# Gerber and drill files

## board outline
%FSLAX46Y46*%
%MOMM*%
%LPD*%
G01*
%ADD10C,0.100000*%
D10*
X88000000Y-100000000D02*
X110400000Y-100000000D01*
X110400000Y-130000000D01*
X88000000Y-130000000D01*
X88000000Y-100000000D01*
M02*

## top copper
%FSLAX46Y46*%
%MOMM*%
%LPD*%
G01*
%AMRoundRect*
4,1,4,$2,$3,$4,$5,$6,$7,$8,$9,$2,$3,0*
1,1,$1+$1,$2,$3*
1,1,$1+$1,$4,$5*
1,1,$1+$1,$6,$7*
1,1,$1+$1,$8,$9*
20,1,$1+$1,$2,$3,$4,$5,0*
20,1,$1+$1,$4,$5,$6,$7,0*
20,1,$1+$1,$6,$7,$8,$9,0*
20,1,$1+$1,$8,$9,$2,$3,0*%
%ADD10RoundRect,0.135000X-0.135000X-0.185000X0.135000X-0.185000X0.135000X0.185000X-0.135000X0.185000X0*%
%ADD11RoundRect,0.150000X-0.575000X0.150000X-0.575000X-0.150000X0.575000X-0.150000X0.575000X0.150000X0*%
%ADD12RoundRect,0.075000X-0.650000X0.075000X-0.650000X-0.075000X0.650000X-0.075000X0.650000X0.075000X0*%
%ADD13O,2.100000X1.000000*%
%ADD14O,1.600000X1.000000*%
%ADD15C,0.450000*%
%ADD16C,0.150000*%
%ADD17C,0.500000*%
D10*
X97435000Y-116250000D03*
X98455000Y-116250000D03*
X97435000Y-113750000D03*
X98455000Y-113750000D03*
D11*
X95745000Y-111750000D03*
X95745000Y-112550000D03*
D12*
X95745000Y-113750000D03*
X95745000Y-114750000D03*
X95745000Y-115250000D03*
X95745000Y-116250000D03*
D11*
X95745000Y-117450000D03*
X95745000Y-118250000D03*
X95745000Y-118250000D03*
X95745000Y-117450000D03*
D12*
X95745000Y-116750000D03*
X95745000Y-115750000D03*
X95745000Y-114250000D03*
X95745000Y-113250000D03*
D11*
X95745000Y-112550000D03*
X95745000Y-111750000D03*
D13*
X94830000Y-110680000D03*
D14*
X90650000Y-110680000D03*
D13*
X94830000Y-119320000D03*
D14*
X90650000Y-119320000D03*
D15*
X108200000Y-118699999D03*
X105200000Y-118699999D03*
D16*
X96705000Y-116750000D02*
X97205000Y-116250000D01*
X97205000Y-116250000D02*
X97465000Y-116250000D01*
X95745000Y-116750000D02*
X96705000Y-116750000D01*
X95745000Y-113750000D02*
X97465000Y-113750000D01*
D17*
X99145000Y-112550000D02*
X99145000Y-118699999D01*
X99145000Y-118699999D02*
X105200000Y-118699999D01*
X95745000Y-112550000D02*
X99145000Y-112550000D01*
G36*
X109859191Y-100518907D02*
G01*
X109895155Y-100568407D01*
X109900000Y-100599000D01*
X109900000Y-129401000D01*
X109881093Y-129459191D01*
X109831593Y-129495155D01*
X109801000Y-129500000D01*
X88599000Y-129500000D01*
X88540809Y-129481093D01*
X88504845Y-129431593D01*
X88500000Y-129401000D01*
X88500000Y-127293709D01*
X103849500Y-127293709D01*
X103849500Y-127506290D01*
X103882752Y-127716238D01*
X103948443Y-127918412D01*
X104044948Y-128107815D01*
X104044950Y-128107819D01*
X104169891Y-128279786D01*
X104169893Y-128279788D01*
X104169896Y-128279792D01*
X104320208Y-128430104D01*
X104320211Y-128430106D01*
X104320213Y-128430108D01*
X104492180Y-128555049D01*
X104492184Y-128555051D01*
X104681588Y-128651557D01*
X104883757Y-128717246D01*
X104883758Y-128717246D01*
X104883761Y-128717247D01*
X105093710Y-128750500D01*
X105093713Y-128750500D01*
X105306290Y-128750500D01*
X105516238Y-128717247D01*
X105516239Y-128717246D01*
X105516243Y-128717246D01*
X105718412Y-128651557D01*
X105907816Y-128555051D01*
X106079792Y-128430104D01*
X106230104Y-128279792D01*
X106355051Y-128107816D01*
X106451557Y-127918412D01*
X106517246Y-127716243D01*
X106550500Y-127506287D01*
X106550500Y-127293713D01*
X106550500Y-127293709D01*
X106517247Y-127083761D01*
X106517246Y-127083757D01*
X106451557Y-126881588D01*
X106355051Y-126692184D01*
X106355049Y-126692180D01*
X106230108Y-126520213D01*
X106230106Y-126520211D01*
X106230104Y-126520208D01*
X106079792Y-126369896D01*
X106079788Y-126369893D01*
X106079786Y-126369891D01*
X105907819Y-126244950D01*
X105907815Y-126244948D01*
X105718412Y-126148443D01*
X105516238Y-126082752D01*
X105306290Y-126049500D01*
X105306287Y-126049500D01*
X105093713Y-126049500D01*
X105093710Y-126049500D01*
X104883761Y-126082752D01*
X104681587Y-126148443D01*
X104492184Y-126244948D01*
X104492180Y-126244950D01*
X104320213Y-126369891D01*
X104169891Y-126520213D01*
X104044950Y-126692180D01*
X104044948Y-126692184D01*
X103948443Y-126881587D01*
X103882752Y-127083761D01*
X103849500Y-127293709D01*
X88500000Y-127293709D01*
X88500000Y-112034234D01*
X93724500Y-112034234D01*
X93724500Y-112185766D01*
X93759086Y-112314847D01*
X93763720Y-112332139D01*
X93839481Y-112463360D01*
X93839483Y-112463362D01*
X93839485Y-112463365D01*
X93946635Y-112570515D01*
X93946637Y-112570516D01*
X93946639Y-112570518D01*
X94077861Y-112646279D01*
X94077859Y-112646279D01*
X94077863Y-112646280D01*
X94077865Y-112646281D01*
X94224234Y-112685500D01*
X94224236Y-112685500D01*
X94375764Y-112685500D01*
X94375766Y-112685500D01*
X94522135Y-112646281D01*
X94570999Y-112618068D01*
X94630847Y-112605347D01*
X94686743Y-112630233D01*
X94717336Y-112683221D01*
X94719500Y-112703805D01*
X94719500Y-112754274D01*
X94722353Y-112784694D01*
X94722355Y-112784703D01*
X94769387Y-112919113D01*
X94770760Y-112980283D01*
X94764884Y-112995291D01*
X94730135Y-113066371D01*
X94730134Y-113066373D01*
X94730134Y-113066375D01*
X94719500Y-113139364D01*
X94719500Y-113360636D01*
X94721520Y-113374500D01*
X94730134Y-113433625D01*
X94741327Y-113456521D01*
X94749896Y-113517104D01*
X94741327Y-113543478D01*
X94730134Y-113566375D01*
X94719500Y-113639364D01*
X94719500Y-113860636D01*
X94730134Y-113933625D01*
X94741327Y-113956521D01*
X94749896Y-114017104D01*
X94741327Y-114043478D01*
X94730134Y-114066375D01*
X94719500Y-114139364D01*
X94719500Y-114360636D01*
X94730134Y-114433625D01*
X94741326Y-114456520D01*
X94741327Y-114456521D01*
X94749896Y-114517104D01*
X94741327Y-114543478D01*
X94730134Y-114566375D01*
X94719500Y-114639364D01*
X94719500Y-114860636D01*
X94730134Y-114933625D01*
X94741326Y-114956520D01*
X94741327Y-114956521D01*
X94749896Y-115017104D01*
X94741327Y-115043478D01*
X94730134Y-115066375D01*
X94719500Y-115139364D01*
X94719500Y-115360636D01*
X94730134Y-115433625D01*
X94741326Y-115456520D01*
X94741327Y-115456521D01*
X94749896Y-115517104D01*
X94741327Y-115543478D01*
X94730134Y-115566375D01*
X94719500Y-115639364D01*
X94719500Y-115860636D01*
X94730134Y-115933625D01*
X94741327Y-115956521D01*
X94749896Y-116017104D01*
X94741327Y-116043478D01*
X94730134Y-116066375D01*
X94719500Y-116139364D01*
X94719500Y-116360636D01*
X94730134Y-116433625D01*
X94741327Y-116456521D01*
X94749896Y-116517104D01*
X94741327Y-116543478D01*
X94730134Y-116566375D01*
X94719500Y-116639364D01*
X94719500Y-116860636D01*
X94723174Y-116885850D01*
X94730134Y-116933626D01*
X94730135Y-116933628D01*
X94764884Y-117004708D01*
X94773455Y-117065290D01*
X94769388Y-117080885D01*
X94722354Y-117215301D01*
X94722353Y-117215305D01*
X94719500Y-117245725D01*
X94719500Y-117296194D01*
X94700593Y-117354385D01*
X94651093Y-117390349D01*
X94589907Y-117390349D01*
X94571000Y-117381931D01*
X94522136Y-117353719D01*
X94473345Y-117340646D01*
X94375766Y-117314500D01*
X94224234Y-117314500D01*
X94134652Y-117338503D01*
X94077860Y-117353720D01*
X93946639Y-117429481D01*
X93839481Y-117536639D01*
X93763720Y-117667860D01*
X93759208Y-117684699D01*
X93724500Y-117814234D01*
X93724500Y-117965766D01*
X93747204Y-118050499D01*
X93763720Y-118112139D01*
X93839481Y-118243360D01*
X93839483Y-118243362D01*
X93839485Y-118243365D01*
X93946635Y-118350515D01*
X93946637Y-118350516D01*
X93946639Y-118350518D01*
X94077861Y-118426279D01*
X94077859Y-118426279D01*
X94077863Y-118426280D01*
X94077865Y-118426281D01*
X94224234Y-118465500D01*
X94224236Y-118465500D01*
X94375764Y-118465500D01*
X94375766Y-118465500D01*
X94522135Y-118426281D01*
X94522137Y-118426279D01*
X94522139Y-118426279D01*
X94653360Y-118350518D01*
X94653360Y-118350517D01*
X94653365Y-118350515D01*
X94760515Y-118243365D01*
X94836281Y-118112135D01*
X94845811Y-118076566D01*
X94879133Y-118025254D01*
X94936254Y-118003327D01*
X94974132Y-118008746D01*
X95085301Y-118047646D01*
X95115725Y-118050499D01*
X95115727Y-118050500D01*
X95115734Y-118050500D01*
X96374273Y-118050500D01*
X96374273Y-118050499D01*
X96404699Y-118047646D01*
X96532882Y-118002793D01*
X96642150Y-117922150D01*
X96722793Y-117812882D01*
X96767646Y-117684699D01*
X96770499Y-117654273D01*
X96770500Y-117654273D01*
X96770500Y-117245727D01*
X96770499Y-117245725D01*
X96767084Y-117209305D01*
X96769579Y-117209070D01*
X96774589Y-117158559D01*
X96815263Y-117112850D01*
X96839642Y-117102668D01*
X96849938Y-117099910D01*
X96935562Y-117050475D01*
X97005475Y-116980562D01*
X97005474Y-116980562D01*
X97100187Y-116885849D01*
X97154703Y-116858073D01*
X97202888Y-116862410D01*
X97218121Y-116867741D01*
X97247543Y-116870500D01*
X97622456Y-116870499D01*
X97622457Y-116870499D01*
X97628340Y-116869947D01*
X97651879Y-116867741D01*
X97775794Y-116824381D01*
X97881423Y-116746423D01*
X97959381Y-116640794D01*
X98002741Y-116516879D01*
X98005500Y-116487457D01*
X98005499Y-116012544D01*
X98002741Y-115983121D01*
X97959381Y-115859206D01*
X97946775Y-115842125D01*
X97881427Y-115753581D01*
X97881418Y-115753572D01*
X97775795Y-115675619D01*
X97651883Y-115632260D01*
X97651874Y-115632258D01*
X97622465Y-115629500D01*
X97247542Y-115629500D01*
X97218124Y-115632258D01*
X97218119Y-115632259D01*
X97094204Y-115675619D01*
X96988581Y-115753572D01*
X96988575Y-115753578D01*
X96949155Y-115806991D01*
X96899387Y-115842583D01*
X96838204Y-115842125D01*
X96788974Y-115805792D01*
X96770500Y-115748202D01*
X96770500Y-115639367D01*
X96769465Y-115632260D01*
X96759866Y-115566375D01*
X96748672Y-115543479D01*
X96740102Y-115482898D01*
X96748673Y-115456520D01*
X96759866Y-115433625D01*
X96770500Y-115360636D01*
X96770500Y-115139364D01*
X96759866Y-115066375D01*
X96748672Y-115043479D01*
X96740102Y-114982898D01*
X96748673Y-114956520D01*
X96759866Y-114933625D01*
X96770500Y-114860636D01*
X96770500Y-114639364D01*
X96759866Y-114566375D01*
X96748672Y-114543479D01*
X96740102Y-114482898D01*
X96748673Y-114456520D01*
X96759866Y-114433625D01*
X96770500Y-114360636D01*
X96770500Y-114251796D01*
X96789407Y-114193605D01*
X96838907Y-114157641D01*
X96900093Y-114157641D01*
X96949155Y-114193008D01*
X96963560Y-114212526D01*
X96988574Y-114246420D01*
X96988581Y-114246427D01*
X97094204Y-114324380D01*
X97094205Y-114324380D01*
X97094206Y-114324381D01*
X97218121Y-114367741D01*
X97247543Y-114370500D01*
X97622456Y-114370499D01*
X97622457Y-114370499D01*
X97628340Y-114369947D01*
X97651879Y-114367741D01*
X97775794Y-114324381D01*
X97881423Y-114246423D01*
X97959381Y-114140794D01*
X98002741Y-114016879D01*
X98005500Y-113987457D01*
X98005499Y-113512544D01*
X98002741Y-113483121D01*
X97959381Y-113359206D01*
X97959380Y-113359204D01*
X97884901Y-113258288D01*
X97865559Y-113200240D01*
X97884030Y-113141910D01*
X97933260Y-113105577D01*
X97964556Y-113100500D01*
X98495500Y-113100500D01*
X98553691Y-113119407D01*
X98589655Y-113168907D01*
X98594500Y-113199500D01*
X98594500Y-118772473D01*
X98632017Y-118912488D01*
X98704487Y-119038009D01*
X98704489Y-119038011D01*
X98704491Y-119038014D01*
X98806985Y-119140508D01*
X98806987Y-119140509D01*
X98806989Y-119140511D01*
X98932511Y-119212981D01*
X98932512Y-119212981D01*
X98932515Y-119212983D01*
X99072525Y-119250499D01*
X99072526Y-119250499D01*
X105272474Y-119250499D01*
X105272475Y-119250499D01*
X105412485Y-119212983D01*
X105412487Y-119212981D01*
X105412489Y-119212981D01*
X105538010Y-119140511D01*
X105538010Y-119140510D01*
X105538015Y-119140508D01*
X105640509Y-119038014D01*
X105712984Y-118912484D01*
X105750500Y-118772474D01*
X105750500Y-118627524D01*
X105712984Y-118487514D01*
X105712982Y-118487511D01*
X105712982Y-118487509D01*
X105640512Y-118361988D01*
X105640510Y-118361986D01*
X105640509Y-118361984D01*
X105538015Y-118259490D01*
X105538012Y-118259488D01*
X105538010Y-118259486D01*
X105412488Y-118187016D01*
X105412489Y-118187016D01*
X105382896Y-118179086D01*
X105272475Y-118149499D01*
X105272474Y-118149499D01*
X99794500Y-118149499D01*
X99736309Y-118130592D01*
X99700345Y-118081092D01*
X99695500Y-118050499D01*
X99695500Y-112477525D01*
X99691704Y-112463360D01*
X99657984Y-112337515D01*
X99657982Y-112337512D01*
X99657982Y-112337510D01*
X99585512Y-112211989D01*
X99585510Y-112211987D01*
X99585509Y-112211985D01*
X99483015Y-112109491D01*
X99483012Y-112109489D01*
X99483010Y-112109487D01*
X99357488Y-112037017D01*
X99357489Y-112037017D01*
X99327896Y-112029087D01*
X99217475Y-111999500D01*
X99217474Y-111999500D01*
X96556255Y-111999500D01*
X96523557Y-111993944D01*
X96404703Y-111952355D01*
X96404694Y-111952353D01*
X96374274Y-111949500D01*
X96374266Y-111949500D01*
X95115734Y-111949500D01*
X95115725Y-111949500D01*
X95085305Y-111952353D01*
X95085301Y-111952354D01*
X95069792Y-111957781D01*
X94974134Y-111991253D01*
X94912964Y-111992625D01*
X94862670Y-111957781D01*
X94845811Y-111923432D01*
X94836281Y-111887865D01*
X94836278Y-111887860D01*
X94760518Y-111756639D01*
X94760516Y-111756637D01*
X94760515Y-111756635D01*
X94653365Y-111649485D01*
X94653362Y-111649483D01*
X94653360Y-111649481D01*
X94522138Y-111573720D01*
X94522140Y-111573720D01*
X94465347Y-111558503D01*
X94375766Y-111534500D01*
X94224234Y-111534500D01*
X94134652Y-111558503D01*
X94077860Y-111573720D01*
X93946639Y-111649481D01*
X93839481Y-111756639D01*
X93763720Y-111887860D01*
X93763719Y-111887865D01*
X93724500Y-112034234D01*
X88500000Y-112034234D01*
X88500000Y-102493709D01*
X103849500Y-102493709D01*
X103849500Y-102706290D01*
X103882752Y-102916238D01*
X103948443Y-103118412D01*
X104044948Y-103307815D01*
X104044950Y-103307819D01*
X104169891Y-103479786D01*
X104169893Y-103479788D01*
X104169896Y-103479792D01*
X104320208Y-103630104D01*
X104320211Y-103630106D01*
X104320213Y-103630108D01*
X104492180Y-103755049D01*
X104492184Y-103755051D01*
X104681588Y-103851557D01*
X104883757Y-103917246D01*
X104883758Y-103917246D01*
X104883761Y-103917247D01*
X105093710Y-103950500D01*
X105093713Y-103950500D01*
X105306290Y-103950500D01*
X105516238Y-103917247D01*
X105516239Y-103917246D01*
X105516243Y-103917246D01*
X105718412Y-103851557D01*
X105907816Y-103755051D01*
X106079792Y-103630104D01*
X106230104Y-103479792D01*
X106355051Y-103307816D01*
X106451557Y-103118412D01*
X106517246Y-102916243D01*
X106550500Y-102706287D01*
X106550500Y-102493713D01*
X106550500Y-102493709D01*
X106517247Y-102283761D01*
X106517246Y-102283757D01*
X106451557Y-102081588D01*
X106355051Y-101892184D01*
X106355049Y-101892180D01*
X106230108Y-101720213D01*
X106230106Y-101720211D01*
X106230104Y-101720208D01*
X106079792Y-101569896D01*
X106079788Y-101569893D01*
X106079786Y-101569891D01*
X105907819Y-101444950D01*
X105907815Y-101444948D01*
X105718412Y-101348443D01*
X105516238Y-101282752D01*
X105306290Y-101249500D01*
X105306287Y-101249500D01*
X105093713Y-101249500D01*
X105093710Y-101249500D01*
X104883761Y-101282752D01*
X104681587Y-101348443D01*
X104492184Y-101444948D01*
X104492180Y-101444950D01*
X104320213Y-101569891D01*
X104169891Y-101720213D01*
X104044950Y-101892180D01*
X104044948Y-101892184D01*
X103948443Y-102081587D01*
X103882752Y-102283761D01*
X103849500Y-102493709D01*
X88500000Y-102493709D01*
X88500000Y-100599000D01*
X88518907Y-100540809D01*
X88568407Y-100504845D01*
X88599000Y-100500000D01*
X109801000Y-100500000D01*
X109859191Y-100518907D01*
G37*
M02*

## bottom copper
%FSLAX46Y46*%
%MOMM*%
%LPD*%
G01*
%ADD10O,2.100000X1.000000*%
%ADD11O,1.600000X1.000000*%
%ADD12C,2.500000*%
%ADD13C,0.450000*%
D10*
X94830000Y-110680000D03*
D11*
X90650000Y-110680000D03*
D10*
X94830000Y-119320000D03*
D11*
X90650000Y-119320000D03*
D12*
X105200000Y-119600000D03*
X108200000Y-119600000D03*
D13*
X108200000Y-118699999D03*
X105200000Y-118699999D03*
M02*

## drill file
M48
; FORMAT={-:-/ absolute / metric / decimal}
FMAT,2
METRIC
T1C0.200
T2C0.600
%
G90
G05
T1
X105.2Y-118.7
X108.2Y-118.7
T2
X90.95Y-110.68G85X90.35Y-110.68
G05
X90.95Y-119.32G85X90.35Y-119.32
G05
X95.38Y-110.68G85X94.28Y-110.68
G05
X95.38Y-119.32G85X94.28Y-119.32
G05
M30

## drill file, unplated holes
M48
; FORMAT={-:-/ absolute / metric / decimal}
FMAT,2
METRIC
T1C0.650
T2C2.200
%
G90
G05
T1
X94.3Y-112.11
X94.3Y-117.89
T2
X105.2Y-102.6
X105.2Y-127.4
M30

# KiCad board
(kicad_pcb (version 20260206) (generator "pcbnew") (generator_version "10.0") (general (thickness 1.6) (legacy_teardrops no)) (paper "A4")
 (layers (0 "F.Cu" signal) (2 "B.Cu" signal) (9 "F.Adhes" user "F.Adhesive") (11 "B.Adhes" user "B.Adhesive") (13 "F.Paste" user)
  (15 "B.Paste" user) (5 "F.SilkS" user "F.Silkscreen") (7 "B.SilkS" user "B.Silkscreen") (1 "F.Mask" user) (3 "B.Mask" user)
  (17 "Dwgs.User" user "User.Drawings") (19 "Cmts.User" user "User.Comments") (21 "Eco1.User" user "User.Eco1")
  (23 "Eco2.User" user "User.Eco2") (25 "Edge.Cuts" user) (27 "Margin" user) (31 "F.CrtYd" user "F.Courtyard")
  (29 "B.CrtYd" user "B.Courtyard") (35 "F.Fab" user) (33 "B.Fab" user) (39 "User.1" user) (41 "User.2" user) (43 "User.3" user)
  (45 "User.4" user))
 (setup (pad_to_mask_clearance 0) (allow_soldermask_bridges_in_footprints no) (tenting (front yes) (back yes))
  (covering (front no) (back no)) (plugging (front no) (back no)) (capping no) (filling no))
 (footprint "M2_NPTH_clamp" (layer "F.Cu") (at 105.2 102.6)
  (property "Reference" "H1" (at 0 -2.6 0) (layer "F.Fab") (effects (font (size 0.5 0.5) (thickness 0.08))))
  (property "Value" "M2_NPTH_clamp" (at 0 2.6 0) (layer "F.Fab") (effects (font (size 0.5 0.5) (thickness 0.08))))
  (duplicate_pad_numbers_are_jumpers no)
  (pad "" np_thru_hole circle (at 0 0) (size 2.2 2.2) (drill 2.2) (layers "*.Cu" "*.Mask")))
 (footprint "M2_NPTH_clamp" (layer "F.Cu") (at 105.2 127.4)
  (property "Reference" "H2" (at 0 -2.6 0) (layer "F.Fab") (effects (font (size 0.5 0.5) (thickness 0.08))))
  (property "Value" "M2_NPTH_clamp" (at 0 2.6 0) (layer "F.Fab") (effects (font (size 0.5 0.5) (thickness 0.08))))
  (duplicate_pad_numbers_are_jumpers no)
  (pad "" np_thru_hole circle (at 0 0) (size 2.2 2.2) (drill 2.2) (layers "*.Cu" "*.Mask")))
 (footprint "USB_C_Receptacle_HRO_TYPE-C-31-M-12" (layer "F.Cu") (at 91.7 115 -90)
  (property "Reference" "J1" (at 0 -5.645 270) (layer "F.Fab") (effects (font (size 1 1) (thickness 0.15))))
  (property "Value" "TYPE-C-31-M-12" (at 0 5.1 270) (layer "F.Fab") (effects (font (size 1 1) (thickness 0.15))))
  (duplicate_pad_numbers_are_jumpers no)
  (pad "" np_thru_hole circle (at -2.89 -2.6 270) (size 0.65 0.65) (drill 0.65) (layers "*.Cu" "*.Mask"))
  (pad "" np_thru_hole circle (at 2.89 -2.6 270) (size 0.65 0.65) (drill 0.65) (layers "*.Cu" "*.Mask"))
  (pad "A1" smd roundrect (at -3.25 -4.045 270) (size 0.6 1.45) (layers "F.Cu" "F.Mask" "F.Paste") (roundrect_rratio 0.25) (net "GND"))
  (pad "A4" smd roundrect (at -2.45 -4.045 270) (size 0.6 1.45) (layers "F.Cu" "F.Mask" "F.Paste") (roundrect_rratio 0.25) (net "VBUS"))
  (pad "A5" smd roundrect (at -1.25 -4.045 270) (size 0.3 1.45) (layers "F.Cu" "F.Mask" "F.Paste") (roundrect_rratio 0.25) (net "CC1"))
  (pad "A6" smd roundrect (at -0.25 -4.045 270) (size 0.3 1.45) (layers "F.Cu" "F.Mask" "F.Paste") (roundrect_rratio 0.25))
  (pad "A7" smd roundrect (at 0.25 -4.045 270) (size 0.3 1.45) (layers "F.Cu" "F.Mask" "F.Paste") (roundrect_rratio 0.25))
  (pad "A8" smd roundrect (at 1.25 -4.045 270) (size 0.3 1.45) (layers "F.Cu" "F.Mask" "F.Paste") (roundrect_rratio 0.25))
  (pad "A9" smd roundrect (at 2.45 -4.045 270) (size 0.6 1.45) (layers "F.Cu" "F.Mask" "F.Paste") (roundrect_rratio 0.25) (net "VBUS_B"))
  (pad "A12" smd roundrect (at 3.25 -4.045 270) (size 0.6 1.45) (layers "F.Cu" "F.Mask" "F.Paste") (roundrect_rratio 0.25) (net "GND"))
  (pad "B1" smd roundrect (at 3.25 -4.045 270) (size 0.6 1.45) (layers "F.Cu" "F.Mask" "F.Paste") (roundrect_rratio 0.25) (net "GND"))
  (pad "B4" smd roundrect (at 2.45 -4.045 270) (size 0.6 1.45) (layers "F.Cu" "F.Mask" "F.Paste") (roundrect_rratio 0.25) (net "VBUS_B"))
  (pad "B5" smd roundrect (at 1.75 -4.045 270) (size 0.3 1.45) (layers "F.Cu" "F.Mask" "F.Paste") (roundrect_rratio 0.25) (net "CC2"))
  (pad "B6" smd roundrect (at 0.75 -4.045 270) (size 0.3 1.45) (layers "F.Cu" "F.Mask" "F.Paste") (roundrect_rratio 0.25))
  (pad "B7" smd roundrect (at -0.75 -4.045 270) (size 0.3 1.45) (layers "F.Cu" "F.Mask" "F.Paste") (roundrect_rratio 0.25))
  (pad "B8" smd roundrect (at -1.75 -4.045 270) (size 0.3 1.45) (layers "F.Cu" "F.Mask" "F.Paste") (roundrect_rratio 0.25))
  (pad "B9" smd roundrect (at -2.45 -4.045 270) (size 0.6 1.45) (layers "F.Cu" "F.Mask" "F.Paste") (roundrect_rratio 0.25) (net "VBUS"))
  (pad "B12" smd roundrect (at -3.25 -4.045 270) (size 0.6 1.45) (layers "F.Cu" "F.Mask" "F.Paste") (roundrect_rratio 0.25) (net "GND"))
  (pad "SH" thru_hole oval (at -4.32 -3.13 270) (size 1 2.1) (drill oval 0.6 1.7) (layers "*.Cu" "*.Mask") (remove_unused_layers no)
   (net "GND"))
  (pad "SH" thru_hole oval (at -4.32 1.05 270) (size 1 1.6) (drill oval 0.6 1.2) (layers "*.Cu" "*.Mask") (remove_unused_layers no)
   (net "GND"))
  (pad "SH" thru_hole oval (at 4.32 -3.13 270) (size 1 2.1) (drill oval 0.6 1.7) (layers "*.Cu" "*.Mask") (remove_unused_layers no)
   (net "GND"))
  (pad "SH" thru_hole oval (at 4.32 1.05 270) (size 1 1.6) (drill oval 0.6 1.2) (layers "*.Cu" "*.Mask") (remove_unused_layers no)
   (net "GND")))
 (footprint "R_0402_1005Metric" (layer "F.Cu") (at 97.945 116.25)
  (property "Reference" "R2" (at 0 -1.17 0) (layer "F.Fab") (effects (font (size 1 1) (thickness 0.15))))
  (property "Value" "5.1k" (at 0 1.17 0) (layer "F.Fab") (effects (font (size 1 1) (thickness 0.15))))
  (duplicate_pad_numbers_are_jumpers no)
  (pad "1" smd roundrect (at -0.51 0) (size 0.54 0.64) (layers "F.Cu" "F.Mask" "F.Paste") (roundrect_rratio 0.25) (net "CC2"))
  (pad "2" smd roundrect (at 0.51 0) (size 0.54 0.64) (layers "F.Cu" "F.Mask" "F.Paste") (roundrect_rratio 0.25) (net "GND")))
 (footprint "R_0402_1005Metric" (layer "F.Cu") (at 97.945 113.75)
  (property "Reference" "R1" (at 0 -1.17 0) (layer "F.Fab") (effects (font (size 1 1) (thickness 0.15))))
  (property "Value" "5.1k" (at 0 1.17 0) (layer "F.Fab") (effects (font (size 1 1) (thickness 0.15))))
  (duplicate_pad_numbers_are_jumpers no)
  (pad "1" smd roundrect (at -0.51 0) (size 0.54 0.64) (layers "F.Cu" "F.Mask" "F.Paste") (roundrect_rratio 0.25) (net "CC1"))
  (pad "2" smd roundrect (at 0.51 0) (size 0.54 0.64) (layers "F.Cu" "F.Mask" "F.Paste") (roundrect_rratio 0.25) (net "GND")))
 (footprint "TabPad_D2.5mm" (layer "B.Cu") (at 105.2 119.6 180)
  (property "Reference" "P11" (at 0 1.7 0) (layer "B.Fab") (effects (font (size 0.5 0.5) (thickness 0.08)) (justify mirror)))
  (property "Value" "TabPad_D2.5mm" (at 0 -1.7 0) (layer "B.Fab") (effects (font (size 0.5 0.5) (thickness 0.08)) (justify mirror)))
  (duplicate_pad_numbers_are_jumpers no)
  (pad "1" smd circle (at 0 0 180) (size 2.5 2.5) (layers "B.Cu" "B.Mask") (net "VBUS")))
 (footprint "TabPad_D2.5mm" (layer "B.Cu") (at 108.2 119.6 180)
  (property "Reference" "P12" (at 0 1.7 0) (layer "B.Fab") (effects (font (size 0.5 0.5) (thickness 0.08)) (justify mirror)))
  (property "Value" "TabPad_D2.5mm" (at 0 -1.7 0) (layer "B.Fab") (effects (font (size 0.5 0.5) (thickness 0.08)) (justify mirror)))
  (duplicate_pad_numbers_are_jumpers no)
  (pad "1" smd circle (at 0 0 180) (size 2.5 2.5) (layers "B.Cu" "B.Mask") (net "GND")))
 (gr_line (start 88 100) (end 110.4 100) (stroke (width 0.1) (type default)) (layer "Edge.Cuts"))
 (gr_line (start 88 130) (end 88 100) (stroke (width 0.1) (type default)) (layer "Edge.Cuts"))
 (gr_line (start 110.4 100) (end 110.4 130) (stroke (width 0.1) (type default)) (layer "Edge.Cuts"))
 (gr_line (start 110.4 130) (end 88 130) (stroke (width 0.1) (type default)) (layer "Edge.Cuts"))
 (via (at 108.2 118.699999) (size 0.45) (drill 0.2) (layers "F.Cu" "B.Cu") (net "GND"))
 (segment (start 95.745 112.55) (end 99.145 112.55) (width 0.5) (layer "F.Cu") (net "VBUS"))
 (segment (start 99.145 118.699999) (end 105.2 118.699999) (width 0.5) (layer "F.Cu") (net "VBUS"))
 (segment (start 99.145 112.55) (end 99.145 118.699999) (width 0.5) (layer "F.Cu") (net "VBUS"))
 (via (at 105.2 118.699999) (size 0.45) (drill 0.2) (layers "F.Cu" "B.Cu") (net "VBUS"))
 (segment (start 95.745 113.75) (end 97.465 113.75) (width 0.15) (layer "F.Cu") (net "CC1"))
 (segment (start 96.705 116.75) (end 97.205 116.25) (width 0.15) (layer "F.Cu") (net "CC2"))
 (segment (start 97.205 116.25) (end 97.465 116.25) (width 0.15) (layer "F.Cu") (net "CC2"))
 (segment (start 95.745 116.75) (end 96.705 116.75) (width 0.15) (layer "F.Cu") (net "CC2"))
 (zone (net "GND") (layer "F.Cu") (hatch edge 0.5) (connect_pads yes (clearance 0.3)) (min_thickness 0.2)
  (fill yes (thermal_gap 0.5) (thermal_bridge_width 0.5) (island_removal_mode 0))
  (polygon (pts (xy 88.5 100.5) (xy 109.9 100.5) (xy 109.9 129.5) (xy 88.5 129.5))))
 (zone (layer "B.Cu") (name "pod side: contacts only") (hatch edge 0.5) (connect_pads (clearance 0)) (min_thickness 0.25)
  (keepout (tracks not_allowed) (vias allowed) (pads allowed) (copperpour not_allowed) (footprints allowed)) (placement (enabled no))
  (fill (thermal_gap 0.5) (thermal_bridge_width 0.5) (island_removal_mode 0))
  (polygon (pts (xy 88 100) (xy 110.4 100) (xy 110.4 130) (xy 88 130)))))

